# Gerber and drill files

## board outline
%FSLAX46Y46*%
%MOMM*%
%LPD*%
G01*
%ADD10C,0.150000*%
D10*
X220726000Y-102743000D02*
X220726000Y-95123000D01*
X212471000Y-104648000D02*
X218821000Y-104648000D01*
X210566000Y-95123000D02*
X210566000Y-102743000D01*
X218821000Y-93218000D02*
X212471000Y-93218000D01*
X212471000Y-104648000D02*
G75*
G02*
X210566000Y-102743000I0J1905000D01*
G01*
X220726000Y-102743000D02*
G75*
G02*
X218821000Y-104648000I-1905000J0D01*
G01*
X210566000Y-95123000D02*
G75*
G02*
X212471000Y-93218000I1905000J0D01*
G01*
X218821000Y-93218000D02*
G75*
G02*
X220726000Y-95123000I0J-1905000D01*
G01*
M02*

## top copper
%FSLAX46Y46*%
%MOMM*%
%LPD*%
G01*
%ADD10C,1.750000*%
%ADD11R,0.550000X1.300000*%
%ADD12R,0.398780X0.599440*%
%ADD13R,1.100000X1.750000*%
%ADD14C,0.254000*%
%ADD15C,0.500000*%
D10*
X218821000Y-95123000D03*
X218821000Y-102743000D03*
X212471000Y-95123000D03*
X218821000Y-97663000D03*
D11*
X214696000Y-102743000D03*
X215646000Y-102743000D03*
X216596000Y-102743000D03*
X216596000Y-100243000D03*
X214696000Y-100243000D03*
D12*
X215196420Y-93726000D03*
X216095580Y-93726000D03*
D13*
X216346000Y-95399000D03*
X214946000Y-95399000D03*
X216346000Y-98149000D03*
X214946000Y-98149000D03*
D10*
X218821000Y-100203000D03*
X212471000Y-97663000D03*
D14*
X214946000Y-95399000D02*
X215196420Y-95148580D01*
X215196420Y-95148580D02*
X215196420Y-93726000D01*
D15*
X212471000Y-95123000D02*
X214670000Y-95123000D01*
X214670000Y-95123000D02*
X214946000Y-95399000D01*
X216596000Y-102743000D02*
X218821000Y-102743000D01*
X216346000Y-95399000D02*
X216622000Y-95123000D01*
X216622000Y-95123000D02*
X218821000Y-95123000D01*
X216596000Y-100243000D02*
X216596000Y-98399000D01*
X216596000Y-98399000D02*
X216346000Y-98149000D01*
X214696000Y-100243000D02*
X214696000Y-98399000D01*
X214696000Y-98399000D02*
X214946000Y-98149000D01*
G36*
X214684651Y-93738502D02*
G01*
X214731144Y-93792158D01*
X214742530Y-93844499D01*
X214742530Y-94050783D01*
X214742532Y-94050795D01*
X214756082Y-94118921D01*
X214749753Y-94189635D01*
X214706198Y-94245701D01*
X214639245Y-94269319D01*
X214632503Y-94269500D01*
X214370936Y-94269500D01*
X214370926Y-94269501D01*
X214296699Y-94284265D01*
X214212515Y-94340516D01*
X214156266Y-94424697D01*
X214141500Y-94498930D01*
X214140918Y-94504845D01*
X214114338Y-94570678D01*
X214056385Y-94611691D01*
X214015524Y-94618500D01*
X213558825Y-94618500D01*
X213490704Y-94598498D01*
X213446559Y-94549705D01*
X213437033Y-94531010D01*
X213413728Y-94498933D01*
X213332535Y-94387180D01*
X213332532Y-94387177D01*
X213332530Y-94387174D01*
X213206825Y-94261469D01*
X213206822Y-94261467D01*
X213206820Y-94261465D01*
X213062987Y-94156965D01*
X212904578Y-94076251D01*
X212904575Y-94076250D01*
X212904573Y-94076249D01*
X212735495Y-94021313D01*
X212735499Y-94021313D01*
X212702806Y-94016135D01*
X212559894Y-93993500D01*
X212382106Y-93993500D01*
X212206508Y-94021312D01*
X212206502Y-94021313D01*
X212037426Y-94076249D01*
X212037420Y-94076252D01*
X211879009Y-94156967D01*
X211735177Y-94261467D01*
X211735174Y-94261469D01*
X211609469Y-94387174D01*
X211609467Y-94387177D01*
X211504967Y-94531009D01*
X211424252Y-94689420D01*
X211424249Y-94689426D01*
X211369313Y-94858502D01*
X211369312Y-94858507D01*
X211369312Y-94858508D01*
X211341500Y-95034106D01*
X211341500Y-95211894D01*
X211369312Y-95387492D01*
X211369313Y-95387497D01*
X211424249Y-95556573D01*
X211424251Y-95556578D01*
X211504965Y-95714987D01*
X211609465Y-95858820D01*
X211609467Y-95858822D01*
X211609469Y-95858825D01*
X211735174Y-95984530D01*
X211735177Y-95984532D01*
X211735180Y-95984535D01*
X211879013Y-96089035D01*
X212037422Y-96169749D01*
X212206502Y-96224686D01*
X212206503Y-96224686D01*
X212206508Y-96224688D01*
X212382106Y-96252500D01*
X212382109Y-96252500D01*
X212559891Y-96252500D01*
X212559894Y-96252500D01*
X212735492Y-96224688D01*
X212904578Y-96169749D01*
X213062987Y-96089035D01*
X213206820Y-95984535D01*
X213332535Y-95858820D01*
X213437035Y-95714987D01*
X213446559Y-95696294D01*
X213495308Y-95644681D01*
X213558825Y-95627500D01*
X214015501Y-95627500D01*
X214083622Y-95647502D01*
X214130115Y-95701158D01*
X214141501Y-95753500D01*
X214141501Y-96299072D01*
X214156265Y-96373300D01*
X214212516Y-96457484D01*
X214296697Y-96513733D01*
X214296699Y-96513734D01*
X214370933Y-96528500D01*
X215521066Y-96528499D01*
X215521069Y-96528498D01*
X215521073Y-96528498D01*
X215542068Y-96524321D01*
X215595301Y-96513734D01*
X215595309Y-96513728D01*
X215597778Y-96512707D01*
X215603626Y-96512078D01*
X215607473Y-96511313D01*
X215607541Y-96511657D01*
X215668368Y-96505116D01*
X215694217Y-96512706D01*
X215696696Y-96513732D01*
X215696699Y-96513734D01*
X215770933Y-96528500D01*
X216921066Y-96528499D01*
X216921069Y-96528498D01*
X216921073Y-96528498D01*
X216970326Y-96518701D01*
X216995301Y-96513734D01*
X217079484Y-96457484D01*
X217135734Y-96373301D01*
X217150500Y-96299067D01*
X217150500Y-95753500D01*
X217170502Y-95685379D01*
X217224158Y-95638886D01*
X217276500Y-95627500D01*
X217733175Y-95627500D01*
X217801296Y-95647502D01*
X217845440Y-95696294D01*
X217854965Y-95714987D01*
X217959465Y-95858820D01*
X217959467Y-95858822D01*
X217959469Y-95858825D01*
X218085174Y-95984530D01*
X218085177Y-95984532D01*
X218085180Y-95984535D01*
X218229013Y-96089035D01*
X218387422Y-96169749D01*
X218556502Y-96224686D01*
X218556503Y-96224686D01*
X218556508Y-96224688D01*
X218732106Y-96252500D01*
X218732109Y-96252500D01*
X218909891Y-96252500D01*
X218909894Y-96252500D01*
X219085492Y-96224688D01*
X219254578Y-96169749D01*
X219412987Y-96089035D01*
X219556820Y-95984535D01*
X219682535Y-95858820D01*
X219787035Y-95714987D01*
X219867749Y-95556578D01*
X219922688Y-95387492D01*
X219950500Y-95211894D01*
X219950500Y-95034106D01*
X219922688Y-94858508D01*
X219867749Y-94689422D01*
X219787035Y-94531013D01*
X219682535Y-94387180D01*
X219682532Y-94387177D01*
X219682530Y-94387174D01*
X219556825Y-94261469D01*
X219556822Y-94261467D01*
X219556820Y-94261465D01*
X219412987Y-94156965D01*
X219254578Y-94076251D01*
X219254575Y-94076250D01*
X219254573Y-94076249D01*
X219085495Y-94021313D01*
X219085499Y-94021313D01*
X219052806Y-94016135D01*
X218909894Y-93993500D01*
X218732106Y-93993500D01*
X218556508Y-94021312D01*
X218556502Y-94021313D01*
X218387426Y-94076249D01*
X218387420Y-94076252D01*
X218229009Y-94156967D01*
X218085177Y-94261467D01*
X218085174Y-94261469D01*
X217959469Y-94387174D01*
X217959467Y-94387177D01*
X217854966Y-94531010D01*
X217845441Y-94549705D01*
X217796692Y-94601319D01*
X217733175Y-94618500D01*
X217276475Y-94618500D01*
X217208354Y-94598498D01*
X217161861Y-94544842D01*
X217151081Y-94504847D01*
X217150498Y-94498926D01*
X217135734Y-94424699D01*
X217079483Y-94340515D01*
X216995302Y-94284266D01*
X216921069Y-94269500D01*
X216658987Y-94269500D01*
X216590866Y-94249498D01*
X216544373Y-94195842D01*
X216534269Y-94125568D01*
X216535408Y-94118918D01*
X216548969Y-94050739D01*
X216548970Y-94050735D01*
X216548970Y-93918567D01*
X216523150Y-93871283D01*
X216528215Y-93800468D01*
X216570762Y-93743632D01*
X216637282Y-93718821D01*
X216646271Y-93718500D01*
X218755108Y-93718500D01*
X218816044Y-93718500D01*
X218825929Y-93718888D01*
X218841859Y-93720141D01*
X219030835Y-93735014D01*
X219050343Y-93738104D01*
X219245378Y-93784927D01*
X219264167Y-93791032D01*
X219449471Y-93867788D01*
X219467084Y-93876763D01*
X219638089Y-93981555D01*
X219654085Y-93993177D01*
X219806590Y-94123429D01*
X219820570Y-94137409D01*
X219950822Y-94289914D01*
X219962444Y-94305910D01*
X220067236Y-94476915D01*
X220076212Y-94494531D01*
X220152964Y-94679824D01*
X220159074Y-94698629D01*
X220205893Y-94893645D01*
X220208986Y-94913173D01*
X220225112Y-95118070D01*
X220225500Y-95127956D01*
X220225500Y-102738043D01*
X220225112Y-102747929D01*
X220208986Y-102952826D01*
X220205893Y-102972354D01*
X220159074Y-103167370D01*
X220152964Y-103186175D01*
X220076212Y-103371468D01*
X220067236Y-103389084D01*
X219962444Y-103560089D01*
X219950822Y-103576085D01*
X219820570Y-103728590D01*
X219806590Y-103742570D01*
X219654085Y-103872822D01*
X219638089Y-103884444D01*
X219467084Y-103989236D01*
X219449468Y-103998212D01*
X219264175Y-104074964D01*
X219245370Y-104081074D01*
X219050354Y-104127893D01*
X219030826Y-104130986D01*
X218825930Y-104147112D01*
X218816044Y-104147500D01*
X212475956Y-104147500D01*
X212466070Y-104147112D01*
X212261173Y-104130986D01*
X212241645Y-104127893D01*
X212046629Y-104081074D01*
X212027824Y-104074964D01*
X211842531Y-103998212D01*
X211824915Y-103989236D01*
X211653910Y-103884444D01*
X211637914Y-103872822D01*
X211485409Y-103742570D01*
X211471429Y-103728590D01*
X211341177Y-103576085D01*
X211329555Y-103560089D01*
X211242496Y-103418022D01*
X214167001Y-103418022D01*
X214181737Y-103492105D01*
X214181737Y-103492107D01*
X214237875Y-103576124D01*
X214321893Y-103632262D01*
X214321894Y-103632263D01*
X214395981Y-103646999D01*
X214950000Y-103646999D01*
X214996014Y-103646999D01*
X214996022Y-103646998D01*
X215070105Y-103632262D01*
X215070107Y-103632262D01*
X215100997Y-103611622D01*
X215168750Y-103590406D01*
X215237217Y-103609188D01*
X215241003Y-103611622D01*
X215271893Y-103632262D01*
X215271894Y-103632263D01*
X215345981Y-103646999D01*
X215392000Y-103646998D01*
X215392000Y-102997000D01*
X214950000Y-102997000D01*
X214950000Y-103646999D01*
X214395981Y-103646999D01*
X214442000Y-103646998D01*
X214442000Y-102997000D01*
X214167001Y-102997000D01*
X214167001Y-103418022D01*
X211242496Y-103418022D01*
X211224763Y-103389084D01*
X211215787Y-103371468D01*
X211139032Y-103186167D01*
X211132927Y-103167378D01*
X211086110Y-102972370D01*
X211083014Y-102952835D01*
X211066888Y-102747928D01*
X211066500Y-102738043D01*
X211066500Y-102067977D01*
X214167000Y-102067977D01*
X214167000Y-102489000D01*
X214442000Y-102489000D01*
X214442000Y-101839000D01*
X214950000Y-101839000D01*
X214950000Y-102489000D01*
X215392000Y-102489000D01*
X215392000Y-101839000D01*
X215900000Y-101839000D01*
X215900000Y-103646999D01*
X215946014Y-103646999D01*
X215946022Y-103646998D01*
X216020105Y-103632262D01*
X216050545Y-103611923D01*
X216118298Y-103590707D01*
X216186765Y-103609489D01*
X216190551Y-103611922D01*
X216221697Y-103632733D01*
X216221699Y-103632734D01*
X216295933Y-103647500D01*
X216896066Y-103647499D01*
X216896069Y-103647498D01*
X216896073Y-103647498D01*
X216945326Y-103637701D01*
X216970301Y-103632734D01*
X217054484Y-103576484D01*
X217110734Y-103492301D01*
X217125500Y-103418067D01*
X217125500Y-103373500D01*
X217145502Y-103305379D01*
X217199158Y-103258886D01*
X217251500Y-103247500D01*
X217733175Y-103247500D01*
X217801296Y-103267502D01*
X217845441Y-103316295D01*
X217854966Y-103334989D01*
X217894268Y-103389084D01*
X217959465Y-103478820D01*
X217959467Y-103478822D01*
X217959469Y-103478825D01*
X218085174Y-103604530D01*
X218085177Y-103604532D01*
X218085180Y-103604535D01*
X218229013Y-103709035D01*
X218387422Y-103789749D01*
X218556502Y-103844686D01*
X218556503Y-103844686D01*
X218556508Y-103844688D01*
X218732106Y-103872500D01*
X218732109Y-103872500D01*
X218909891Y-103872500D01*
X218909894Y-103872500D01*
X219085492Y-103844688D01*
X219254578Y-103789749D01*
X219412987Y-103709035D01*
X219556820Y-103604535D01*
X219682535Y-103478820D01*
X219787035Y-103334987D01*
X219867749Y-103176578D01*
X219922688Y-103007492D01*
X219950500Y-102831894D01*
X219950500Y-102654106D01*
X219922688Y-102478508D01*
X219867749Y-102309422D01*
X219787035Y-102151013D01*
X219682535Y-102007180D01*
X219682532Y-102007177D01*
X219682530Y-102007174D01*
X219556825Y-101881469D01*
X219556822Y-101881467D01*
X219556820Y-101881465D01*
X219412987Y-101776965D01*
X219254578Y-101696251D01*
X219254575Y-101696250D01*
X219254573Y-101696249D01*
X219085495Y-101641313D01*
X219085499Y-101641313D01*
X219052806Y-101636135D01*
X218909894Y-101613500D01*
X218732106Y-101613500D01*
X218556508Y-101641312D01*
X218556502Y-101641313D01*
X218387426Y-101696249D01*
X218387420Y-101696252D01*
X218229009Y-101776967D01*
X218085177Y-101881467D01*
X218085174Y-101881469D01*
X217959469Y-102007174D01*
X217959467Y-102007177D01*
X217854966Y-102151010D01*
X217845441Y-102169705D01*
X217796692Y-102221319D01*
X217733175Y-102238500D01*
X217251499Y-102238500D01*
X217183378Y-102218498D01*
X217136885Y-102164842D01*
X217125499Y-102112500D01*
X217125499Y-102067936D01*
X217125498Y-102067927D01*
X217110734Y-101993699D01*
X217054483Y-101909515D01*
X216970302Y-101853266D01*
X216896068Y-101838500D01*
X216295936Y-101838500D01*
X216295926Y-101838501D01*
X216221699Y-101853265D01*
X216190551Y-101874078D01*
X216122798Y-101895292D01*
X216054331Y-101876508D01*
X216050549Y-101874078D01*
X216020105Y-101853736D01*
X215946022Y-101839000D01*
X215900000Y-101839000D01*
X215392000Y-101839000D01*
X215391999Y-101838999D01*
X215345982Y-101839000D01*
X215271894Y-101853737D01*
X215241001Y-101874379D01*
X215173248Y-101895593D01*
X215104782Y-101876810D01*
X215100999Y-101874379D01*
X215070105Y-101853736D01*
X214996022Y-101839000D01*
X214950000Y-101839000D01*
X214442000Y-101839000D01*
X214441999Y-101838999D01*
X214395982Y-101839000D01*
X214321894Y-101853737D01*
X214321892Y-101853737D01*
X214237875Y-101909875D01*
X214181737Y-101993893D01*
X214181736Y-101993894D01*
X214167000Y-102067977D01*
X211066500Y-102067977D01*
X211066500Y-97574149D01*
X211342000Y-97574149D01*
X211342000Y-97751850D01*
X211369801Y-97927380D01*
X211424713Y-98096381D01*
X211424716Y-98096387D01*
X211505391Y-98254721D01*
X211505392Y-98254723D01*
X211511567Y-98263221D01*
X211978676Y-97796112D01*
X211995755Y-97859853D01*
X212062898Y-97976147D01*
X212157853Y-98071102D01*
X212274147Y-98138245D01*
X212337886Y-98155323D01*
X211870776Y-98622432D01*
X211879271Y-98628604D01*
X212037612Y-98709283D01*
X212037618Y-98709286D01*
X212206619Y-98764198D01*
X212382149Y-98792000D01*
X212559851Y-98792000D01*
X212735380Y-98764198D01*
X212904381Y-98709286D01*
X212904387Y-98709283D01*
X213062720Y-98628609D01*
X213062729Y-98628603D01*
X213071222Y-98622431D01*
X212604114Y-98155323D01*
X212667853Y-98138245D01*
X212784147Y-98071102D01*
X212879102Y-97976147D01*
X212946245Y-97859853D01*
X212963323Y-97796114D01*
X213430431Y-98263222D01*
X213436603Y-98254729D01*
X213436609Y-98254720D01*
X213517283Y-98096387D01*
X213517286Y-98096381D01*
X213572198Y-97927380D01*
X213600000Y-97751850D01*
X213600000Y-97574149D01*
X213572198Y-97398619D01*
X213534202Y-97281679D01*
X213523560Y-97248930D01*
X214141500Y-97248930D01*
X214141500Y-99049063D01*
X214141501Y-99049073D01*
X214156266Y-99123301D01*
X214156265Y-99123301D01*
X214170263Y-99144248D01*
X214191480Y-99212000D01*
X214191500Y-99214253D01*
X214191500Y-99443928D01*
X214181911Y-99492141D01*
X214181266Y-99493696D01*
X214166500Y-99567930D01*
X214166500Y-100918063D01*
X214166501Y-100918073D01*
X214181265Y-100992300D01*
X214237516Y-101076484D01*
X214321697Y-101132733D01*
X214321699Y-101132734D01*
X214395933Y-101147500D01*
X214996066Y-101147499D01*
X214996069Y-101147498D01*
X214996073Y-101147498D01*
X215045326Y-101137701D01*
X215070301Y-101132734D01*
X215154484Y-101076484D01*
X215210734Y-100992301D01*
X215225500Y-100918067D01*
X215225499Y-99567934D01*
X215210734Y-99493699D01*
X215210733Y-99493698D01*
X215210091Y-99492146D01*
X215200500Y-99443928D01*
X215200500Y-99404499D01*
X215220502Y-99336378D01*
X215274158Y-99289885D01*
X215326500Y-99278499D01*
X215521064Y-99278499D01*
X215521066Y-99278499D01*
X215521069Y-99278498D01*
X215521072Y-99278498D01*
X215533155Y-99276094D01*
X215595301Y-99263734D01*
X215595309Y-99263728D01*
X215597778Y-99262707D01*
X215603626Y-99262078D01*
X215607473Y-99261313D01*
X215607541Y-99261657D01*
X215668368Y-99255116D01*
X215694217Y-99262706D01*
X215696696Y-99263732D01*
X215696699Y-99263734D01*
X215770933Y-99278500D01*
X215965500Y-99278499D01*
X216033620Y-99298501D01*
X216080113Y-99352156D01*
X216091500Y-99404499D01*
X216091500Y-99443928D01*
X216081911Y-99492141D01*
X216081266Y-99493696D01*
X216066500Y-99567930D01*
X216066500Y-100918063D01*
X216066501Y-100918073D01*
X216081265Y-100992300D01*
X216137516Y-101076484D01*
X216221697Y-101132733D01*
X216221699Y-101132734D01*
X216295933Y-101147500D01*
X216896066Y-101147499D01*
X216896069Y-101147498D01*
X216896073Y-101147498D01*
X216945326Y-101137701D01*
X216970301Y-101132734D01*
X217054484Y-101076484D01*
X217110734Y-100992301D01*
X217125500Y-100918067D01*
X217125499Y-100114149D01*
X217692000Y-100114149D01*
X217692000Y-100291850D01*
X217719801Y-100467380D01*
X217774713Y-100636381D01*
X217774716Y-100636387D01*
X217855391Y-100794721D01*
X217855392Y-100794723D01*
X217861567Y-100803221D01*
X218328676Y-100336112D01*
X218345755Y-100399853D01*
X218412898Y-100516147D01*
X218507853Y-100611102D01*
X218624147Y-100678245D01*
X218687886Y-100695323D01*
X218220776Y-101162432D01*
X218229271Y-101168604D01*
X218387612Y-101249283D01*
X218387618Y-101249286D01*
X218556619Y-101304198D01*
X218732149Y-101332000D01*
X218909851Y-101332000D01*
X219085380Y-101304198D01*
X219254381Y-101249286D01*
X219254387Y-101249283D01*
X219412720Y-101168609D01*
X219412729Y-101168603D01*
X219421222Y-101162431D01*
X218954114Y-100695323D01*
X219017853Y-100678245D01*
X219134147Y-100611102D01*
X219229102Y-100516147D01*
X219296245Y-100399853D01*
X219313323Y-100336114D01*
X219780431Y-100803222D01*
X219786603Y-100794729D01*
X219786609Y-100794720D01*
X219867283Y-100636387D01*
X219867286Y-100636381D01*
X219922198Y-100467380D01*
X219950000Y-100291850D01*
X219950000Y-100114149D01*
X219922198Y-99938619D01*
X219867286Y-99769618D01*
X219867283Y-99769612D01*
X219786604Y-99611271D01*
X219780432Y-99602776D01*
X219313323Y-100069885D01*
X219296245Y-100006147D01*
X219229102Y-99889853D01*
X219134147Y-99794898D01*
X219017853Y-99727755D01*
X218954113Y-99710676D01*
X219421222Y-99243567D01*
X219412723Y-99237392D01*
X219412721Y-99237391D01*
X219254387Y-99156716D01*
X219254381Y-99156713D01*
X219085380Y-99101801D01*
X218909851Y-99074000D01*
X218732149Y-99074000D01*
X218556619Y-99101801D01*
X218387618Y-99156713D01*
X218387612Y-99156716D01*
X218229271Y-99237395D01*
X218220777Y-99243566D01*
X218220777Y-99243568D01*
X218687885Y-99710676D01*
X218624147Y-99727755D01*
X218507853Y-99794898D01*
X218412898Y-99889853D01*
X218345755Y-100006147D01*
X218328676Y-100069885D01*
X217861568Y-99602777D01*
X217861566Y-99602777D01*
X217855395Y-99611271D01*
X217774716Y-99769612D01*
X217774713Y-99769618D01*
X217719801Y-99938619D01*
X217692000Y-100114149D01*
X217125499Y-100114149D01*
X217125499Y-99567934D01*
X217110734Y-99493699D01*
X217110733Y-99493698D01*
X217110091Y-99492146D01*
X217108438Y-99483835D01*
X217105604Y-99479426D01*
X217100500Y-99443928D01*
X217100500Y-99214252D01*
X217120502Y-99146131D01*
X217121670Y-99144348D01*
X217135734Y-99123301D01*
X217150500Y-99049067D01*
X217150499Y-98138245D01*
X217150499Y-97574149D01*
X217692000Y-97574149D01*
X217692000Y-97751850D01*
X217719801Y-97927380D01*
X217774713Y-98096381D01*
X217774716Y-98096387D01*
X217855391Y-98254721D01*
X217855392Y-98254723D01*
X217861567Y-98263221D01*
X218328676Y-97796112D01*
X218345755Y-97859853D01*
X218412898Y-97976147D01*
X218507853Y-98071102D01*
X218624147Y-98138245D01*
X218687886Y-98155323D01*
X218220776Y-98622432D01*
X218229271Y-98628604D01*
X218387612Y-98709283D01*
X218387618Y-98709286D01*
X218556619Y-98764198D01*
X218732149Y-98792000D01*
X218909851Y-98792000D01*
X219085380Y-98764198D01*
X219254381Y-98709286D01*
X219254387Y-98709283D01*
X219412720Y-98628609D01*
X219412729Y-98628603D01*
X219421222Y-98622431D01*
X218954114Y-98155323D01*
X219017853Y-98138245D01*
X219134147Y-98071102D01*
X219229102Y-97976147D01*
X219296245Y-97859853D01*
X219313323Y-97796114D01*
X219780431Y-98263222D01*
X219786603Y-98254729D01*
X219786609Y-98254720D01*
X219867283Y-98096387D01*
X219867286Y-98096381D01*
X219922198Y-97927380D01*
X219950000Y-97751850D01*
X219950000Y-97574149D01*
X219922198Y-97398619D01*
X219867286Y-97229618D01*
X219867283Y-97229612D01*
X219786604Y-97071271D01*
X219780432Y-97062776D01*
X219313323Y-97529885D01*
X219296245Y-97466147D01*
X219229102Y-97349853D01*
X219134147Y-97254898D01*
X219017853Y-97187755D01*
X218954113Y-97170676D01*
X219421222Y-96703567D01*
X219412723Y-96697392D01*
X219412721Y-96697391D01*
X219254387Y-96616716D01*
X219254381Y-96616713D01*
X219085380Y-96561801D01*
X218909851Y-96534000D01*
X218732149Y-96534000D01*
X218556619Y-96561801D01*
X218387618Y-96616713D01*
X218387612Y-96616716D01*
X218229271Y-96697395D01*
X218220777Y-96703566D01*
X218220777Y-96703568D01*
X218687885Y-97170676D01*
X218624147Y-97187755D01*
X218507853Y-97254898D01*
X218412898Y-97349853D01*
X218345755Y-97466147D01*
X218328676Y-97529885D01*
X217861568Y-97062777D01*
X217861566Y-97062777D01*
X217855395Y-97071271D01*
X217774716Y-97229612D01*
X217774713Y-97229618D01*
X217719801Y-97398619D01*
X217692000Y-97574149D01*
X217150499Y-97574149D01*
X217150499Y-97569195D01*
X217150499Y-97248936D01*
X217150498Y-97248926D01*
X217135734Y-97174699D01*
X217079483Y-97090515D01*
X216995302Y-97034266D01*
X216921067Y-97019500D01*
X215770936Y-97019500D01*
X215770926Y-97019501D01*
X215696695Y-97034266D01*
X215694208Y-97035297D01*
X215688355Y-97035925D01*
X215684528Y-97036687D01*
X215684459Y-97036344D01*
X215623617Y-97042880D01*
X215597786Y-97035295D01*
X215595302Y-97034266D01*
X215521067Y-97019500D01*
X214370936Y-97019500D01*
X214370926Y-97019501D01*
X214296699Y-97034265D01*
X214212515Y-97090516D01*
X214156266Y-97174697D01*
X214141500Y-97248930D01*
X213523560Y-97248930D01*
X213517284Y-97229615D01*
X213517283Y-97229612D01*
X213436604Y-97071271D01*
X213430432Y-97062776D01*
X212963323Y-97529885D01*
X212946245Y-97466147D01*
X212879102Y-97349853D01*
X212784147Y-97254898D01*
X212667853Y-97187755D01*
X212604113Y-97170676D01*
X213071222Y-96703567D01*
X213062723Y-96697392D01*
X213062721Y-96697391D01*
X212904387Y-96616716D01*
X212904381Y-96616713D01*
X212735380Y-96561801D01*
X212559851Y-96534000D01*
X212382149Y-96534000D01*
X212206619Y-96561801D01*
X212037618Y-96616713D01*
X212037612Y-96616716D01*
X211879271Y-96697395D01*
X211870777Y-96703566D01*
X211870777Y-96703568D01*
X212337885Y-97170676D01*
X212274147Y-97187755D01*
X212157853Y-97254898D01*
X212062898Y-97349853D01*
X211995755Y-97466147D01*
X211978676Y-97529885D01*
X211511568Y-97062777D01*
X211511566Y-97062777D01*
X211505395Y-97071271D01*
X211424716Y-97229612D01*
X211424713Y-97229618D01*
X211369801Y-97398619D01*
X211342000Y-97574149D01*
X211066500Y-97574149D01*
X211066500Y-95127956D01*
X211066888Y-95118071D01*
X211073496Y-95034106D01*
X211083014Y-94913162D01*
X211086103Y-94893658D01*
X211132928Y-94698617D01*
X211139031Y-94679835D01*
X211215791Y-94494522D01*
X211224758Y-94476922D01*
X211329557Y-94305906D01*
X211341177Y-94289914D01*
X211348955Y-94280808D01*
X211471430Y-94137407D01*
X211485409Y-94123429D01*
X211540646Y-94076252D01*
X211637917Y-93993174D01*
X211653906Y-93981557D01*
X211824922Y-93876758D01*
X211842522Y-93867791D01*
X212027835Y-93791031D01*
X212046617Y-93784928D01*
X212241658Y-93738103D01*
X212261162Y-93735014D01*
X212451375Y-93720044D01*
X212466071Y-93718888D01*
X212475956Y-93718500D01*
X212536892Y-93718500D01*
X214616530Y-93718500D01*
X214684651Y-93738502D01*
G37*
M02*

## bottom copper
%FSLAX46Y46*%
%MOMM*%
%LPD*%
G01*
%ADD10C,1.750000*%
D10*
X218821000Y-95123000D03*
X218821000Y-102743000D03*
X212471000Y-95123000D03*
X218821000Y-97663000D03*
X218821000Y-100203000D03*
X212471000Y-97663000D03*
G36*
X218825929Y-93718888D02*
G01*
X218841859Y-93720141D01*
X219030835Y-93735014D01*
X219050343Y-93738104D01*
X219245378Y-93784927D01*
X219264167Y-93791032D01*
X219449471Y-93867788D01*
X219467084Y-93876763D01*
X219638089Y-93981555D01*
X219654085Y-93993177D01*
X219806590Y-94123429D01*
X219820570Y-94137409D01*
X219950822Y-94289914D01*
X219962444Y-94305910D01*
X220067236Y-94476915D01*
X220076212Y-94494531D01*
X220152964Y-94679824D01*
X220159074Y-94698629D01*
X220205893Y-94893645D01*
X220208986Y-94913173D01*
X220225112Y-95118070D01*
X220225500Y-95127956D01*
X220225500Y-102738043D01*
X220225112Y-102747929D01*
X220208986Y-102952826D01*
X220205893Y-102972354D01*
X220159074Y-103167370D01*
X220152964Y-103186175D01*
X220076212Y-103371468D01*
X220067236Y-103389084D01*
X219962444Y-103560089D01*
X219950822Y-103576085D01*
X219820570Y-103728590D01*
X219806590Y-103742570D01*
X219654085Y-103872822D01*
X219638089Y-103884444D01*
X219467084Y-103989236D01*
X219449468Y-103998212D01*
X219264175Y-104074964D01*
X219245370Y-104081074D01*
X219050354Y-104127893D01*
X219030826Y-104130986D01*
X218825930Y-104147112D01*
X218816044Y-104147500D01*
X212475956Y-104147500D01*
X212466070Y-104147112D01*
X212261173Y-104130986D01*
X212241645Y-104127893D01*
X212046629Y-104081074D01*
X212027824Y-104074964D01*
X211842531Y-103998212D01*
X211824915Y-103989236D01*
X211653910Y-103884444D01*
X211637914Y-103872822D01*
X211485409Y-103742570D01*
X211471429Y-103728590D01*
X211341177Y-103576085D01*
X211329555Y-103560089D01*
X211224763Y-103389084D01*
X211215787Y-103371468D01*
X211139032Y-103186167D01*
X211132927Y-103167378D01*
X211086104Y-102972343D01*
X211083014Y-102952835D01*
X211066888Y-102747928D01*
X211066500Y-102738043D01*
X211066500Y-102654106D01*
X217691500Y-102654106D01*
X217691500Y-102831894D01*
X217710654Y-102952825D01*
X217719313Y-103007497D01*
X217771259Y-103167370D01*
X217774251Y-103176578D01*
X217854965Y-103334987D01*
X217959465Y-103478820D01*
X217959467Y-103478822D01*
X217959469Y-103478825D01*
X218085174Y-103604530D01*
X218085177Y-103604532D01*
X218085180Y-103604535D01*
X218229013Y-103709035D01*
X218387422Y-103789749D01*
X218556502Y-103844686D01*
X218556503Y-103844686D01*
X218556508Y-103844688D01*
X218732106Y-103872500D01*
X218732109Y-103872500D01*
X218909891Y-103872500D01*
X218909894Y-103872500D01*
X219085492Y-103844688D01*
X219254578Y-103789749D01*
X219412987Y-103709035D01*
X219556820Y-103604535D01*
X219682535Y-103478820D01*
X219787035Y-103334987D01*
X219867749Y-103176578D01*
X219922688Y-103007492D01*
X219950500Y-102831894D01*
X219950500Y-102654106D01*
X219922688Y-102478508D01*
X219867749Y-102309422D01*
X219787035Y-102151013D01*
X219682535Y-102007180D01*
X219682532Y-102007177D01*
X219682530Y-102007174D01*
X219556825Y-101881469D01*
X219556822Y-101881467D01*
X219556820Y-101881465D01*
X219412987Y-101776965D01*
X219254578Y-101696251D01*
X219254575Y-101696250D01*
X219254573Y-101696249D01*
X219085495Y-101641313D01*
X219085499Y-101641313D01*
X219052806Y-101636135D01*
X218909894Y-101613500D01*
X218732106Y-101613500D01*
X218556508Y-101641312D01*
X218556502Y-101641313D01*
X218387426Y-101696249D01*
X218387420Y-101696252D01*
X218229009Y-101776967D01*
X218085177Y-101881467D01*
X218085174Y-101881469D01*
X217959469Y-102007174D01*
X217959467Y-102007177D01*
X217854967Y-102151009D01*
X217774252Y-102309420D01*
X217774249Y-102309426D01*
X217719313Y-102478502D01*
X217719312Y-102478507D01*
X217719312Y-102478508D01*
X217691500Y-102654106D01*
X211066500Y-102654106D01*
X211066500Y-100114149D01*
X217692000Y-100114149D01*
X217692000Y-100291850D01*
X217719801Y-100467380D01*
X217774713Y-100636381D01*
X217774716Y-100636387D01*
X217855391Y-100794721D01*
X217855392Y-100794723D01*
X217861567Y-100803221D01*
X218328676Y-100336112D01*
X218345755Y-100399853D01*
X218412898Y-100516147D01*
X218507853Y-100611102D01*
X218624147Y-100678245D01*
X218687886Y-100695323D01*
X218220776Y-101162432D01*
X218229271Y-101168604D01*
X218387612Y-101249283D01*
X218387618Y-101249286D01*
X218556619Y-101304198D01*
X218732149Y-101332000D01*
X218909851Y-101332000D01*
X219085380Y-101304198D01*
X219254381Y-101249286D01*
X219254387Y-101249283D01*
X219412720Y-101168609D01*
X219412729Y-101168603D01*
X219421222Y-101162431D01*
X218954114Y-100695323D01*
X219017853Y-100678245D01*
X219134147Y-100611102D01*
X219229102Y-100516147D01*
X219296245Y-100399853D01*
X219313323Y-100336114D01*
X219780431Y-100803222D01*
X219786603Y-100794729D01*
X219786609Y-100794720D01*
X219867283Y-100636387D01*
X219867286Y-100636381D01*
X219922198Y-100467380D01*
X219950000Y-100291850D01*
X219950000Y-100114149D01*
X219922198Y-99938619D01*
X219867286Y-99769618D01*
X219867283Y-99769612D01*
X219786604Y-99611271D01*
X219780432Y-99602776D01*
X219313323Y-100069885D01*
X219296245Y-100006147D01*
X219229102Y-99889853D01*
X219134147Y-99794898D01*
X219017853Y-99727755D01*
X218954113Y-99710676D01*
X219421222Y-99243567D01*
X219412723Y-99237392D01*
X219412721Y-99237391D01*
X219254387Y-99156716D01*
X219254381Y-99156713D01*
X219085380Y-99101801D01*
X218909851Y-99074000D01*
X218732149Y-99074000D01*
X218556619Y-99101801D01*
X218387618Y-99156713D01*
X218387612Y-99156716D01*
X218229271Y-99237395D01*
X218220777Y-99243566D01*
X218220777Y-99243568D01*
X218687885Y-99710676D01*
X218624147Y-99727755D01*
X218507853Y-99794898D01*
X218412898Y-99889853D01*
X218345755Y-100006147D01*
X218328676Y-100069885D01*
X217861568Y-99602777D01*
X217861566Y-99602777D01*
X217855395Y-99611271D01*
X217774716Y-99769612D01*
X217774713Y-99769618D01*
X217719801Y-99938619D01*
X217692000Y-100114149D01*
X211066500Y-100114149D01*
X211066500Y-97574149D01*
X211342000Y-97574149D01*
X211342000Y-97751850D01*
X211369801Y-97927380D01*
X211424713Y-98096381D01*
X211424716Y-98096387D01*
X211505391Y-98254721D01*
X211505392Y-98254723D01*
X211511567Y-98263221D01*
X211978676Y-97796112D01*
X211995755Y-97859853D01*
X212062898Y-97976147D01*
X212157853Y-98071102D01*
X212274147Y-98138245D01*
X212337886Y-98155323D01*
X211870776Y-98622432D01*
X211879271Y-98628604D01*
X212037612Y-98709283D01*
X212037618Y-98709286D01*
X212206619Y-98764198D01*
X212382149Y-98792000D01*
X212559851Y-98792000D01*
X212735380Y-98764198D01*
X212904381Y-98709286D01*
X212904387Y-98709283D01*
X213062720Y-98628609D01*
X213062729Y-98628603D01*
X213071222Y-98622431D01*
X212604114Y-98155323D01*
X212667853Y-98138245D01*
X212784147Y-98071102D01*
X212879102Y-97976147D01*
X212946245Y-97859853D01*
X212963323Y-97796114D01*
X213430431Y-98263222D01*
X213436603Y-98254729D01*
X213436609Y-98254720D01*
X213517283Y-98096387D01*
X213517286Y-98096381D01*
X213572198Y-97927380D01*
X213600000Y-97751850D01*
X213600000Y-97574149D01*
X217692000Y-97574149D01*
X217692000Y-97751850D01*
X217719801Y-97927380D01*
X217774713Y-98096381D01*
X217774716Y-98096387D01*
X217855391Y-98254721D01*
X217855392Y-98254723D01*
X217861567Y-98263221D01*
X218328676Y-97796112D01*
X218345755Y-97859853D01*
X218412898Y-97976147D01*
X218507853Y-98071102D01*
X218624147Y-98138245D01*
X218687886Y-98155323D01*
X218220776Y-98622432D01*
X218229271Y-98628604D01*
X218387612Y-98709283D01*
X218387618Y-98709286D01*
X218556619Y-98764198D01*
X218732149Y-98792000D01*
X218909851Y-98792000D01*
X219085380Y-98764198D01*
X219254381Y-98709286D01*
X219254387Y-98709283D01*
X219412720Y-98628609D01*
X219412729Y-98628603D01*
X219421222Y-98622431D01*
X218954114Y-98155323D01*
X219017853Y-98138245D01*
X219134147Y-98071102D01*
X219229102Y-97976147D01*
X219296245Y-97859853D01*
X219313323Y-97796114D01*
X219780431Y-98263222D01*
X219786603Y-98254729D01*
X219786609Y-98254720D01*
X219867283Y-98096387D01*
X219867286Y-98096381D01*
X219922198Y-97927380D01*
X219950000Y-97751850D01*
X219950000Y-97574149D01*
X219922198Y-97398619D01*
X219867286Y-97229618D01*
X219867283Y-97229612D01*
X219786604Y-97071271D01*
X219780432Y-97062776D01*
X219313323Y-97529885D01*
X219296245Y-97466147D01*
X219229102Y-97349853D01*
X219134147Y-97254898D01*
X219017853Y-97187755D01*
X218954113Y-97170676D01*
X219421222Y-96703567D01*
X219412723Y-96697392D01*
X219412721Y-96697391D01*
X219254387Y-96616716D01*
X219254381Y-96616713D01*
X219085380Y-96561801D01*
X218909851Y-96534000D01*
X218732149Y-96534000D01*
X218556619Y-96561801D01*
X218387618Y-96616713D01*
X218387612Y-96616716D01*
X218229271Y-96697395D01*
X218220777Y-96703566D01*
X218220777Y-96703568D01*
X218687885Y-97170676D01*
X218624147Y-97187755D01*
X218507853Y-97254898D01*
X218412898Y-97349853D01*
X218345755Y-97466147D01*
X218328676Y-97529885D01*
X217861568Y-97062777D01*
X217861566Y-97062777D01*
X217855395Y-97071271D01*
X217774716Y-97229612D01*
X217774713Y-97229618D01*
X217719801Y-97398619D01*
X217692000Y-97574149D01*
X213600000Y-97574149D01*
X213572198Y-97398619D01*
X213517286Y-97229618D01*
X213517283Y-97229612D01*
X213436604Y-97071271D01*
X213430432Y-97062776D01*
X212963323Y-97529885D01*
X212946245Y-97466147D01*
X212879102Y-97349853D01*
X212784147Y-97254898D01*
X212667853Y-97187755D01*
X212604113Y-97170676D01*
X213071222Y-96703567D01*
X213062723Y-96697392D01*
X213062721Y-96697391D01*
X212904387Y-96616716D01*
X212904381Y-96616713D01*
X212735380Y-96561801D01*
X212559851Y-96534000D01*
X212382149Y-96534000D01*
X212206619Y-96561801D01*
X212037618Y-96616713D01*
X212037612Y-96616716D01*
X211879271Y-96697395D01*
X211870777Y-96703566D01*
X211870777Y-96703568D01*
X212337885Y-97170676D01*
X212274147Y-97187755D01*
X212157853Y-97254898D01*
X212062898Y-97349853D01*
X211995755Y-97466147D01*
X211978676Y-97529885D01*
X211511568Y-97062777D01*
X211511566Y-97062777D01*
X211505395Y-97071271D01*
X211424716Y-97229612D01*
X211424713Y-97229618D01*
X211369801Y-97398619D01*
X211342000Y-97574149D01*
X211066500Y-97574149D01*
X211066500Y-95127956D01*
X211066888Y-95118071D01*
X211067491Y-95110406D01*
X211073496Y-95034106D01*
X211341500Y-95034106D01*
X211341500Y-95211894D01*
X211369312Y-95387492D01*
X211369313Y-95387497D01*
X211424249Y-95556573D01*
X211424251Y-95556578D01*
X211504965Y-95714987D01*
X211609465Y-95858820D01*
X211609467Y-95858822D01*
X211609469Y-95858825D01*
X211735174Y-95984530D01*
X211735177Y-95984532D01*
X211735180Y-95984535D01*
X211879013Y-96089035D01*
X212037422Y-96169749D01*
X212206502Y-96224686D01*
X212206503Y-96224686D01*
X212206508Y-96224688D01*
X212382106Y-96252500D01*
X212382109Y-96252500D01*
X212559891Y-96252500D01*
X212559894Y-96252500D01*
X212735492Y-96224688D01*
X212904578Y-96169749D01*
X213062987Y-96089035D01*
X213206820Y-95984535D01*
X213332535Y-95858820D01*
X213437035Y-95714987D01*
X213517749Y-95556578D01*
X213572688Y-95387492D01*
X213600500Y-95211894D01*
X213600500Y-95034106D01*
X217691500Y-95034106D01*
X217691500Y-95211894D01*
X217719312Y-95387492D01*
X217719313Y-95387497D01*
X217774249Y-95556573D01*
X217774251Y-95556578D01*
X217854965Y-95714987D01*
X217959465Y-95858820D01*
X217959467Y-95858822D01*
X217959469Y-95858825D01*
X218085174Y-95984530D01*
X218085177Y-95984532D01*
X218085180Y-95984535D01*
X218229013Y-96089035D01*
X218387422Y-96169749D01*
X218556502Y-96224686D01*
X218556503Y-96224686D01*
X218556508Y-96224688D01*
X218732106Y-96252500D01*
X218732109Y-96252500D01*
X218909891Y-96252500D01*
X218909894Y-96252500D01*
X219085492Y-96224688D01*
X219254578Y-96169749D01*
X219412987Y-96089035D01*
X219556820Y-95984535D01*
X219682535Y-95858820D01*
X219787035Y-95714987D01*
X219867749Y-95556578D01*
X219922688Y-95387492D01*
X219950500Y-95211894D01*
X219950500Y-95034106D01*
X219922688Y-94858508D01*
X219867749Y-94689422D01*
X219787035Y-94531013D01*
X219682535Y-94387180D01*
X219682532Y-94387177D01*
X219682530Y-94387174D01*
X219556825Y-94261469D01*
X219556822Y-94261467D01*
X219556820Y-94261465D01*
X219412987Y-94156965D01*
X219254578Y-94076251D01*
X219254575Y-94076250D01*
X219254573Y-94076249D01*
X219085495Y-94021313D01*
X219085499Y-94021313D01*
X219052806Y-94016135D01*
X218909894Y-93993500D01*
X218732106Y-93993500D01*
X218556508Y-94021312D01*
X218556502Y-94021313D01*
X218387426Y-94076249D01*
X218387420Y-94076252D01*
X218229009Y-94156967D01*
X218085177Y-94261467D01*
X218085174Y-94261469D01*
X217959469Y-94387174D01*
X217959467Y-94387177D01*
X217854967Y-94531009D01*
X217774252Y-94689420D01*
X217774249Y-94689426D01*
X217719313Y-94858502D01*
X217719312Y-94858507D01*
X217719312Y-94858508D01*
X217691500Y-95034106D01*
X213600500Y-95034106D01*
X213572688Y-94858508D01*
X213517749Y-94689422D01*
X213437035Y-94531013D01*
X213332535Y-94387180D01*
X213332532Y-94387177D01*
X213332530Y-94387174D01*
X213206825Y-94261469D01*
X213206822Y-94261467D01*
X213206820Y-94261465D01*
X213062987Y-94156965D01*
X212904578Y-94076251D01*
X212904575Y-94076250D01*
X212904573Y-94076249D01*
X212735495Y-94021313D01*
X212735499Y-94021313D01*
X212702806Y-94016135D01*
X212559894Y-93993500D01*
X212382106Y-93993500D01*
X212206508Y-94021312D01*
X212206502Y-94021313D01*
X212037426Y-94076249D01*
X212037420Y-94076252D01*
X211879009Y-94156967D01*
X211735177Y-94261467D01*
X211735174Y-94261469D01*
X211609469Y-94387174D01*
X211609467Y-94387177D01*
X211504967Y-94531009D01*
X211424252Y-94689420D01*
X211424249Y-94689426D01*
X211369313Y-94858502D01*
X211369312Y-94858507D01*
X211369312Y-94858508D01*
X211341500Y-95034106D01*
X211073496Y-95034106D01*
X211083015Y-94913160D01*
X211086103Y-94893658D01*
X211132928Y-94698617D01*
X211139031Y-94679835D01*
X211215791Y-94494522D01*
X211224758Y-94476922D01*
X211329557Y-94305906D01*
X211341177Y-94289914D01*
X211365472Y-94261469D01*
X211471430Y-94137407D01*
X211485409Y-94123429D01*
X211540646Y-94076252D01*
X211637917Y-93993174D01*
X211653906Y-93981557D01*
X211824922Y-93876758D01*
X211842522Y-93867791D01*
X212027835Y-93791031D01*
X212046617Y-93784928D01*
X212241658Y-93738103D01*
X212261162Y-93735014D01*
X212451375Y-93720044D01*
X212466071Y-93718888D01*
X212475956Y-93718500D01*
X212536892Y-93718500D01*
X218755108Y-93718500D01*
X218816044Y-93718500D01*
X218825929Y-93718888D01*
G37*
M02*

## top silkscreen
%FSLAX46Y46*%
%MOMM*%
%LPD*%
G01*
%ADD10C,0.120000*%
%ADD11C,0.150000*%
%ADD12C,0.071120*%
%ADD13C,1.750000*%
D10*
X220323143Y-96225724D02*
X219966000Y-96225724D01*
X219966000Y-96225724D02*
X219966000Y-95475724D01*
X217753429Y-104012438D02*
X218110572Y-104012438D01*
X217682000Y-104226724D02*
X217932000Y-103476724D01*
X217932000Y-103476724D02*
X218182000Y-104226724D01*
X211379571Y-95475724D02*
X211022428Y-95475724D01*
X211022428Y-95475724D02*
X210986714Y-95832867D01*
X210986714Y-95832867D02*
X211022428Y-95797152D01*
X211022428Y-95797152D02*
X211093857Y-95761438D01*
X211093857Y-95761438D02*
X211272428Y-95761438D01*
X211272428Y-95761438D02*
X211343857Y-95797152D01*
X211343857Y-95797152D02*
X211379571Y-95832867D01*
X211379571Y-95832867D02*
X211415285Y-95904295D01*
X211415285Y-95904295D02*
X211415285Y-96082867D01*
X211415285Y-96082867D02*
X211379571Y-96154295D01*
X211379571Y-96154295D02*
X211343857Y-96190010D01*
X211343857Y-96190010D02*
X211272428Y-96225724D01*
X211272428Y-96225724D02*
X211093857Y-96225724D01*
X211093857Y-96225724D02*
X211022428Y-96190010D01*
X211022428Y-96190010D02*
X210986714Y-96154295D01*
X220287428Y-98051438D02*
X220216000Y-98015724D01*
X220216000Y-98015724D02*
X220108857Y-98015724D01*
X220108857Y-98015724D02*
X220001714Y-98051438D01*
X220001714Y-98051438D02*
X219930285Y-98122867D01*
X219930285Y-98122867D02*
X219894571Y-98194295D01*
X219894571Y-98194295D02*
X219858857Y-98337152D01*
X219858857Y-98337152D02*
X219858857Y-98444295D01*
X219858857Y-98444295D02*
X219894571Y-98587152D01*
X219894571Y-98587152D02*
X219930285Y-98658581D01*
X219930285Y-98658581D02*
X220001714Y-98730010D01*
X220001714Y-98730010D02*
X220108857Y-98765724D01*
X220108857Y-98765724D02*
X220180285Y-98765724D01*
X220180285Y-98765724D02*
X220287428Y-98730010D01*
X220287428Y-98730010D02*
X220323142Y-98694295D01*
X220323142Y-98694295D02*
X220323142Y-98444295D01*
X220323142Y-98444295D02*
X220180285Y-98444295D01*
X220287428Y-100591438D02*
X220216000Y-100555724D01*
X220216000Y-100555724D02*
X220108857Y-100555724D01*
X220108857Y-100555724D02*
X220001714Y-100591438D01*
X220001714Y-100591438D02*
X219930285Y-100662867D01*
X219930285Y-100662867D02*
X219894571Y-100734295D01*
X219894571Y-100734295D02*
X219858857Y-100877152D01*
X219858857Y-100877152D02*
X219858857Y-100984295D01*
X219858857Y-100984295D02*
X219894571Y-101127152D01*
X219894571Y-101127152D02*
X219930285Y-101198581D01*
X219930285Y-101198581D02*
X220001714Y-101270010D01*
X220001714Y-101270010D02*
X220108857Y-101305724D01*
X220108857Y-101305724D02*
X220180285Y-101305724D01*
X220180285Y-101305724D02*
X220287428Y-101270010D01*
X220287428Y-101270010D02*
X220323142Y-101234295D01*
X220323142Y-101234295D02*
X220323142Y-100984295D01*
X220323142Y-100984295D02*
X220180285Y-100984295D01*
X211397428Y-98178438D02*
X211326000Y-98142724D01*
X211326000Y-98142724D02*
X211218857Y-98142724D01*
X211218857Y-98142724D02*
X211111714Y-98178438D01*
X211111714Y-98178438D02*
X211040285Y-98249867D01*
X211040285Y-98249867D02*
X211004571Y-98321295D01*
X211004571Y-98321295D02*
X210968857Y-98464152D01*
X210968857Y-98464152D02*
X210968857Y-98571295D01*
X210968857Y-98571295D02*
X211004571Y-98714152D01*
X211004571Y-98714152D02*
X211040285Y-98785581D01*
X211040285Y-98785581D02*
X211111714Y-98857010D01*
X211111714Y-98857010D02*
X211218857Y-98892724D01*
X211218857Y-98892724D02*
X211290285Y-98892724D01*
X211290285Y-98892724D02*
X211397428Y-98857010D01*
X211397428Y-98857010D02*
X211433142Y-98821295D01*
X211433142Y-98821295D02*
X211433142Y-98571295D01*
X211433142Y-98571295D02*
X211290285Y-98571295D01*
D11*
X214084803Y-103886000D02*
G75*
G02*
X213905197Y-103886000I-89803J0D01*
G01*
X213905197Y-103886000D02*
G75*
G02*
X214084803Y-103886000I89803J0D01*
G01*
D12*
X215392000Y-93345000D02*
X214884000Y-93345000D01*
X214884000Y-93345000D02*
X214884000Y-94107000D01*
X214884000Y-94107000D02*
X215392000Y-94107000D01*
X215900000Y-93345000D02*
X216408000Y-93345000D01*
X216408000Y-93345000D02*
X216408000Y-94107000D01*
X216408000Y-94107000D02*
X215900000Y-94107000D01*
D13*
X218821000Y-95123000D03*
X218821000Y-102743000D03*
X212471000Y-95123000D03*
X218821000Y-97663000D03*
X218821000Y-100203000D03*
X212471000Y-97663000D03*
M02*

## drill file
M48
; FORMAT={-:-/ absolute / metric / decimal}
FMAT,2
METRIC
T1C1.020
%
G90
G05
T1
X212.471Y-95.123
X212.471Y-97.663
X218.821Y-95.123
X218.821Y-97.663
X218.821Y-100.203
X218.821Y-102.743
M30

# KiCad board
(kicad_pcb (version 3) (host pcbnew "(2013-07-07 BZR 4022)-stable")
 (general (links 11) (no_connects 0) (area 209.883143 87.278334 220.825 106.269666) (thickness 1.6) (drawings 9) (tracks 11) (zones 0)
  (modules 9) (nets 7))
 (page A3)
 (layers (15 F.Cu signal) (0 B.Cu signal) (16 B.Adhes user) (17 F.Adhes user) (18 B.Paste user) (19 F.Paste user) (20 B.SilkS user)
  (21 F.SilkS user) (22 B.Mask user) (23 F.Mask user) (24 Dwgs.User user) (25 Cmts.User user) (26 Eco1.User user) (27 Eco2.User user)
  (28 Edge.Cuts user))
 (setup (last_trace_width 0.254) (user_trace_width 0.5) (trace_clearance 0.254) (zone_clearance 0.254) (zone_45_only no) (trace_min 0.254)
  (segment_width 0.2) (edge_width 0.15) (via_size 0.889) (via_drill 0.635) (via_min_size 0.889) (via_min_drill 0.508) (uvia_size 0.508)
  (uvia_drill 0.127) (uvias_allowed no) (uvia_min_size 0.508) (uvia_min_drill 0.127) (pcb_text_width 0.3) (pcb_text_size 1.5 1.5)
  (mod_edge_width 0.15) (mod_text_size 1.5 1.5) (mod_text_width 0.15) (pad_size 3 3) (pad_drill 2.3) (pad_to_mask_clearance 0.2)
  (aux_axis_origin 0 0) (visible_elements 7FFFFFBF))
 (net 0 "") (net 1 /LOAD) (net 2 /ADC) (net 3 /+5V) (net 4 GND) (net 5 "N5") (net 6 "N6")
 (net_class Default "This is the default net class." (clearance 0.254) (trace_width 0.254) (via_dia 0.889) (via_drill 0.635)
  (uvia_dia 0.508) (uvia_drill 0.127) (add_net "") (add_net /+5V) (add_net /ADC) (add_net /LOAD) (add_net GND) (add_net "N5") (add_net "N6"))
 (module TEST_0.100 (layer F.Cu) (at 218.821 95.123)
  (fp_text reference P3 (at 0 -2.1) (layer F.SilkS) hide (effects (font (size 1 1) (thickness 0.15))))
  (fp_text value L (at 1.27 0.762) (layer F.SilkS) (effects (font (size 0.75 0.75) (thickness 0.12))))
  (pad 1 thru_hole circle (at 0 0) (size 1.75 1.75) (drill 1.02) (layers *.Cu *.Mask F.SilkS) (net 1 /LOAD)))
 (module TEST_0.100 (layer F.Cu) (at 218.821 102.743)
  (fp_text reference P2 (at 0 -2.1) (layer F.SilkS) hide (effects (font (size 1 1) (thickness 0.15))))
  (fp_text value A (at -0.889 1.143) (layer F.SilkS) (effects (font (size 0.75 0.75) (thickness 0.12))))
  (pad 1 thru_hole circle (at 0 0) (size 1.75 1.75) (drill 1.02) (layers *.Cu *.Mask F.SilkS) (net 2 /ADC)))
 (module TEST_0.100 (layer F.Cu) (at 212.471 95.123)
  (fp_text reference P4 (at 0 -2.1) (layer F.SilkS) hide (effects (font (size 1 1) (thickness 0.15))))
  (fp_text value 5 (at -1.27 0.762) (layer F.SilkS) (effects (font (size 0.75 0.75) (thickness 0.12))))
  (pad 1 thru_hole circle (at 0 0) (size 1.75 1.75) (drill 1.02) (layers *.Cu *.Mask F.SilkS) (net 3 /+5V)))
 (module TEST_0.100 (layer F.Cu) (at 218.821 97.663)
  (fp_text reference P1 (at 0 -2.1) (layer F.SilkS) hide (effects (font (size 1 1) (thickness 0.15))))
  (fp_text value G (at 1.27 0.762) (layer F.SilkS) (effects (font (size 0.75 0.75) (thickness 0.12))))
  (pad 1 thru_hole circle (at 0 0) (size 1.75 1.75) (drill 1.02) (layers *.Cu *.Mask F.SilkS) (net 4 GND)))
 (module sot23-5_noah (layer F.Cu) (at 215.646 102.743 90)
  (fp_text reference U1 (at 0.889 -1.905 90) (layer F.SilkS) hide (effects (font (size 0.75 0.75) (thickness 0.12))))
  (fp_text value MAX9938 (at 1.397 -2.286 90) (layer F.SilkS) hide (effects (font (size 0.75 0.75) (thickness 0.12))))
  (fp_circle (center -1.143 -1.651) (end -1.0795 -1.5875) (layer F.SilkS) (width 0.15))
  (pad 1 smd rect (at 0 -0.95 90) (size 1.3 0.55) (layers F.Cu F.Paste F.Mask) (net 4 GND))
  (pad 2 smd rect (at 0 0 90) (size 1.3 0.55) (layers F.Cu F.Paste F.Mask) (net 4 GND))
  (pad 3 smd rect (at 0 0.95 90) (size 1.3 0.55) (layers F.Cu F.Paste F.Mask) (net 2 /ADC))
  (pad 4 smd rect (at 2.5 0.95 90) (size 1.3 0.55) (layers F.Cu F.Paste F.Mask) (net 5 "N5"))
  (pad 5 smd rect (at 2.5 -0.95 90) (size 1.3 0.55) (layers F.Cu F.Paste F.Mask) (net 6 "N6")))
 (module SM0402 (layer F.Cu) (at 215.646 93.726)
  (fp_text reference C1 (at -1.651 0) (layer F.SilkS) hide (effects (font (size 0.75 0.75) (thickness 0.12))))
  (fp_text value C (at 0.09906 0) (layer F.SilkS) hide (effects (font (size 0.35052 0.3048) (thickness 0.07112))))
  (fp_line (start -0.254 -0.381) (end -0.762 -0.381) (layer F.SilkS) (width 0.07112))
  (fp_line (start -0.762 -0.381) (end -0.762 0.381) (layer F.SilkS) (width 0.07112))
  (fp_line (start -0.762 0.381) (end -0.254 0.381) (layer F.SilkS) (width 0.07112))
  (fp_line (start 0.254 -0.381) (end 0.762 -0.381) (layer F.SilkS) (width 0.07112))
  (fp_line (start 0.762 -0.381) (end 0.762 0.381) (layer F.SilkS) (width 0.07112))
  (fp_line (start 0.762 0.381) (end 0.254 0.381) (layer F.SilkS) (width 0.07112))
  (pad 1 smd rect (at -0.44958 0) (size 0.39878 0.59944) (layers F.Cu F.Paste F.Mask) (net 3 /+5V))
  (pad 2 smd rect (at 0.44958 0) (size 0.39878 0.59944) (layers F.Cu F.Paste F.Mask) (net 4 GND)))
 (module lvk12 (layer F.Cu) (at 215.646 96.774 270)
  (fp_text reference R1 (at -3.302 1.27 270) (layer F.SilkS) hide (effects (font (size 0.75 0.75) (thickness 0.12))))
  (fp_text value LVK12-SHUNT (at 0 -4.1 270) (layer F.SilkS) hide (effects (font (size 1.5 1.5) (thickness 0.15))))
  (pad 1 smd rect (at -1.375 -0.7 270) (size 1.75 1.1) (layers F.Cu F.Paste F.Mask) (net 1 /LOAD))
  (pad 2 smd rect (at -1.375 0.7 270) (size 1.75 1.1) (layers F.Cu F.Paste F.Mask) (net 3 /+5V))
  (pad 4 smd rect (at 1.375 -0.7 270) (size 1.75 1.1) (layers F.Cu F.Paste F.Mask) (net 5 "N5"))
  (pad 3 smd rect (at 1.375 0.7 270) (size 1.75 1.1) (layers F.Cu F.Paste F.Mask) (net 6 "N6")))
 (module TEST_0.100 (layer F.Cu) (at 218.821 100.203)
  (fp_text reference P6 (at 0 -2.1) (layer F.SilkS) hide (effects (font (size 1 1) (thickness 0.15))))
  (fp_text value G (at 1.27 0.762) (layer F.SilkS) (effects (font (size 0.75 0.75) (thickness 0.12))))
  (pad 1 thru_hole circle (at 0 0) (size 1.75 1.75) (drill 1.02) (layers *.Cu *.Mask F.SilkS) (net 4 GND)))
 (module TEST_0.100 (layer F.Cu) (at 212.471 97.663)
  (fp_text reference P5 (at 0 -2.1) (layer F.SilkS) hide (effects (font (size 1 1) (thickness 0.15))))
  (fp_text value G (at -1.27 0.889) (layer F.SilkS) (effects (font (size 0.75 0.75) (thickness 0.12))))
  (pad 1 thru_hole circle (at 0 0) (size 1.75 1.75) (drill 1.02) (layers *.Cu *.Mask F.SilkS) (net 4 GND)))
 (gr_line (start 220.726 102.743) (end 220.726 95.123) (angle 90) (layer Edge.Cuts) (width 0.15))
 (gr_line (start 212.471 104.648) (end 218.821 104.648) (angle 90) (layer Edge.Cuts) (width 0.15))
 (gr_line (start 210.566 95.123) (end 210.566 102.743) (angle 90) (layer Edge.Cuts) (width 0.15))
 (gr_line (start 218.821 93.218) (end 212.471 93.218) (angle 90) (layer Edge.Cuts) (width 0.15))
 (gr_arc (start 212.471 102.743) (end 212.471 104.648) (angle 90) (layer Edge.Cuts) (width 0.15))
 (gr_arc (start 218.821 102.743) (end 220.726 102.743) (angle 90) (layer Edge.Cuts) (width 0.15))
 (gr_arc (start 212.471 95.123) (end 210.566 95.123) (angle 90) (layer Edge.Cuts) (width 0.15))
 (gr_arc (start 218.821 95.123) (end 218.821 93.218) (angle 90) (layer Edge.Cuts) (width 0.15))
 (segment (start 214.946 95.399) (end 215.19642 95.14858) (width 0.254) (layer F.Cu) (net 3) (status C00000))
 (segment (start 215.19642 95.14858) (end 215.19642 93.726) (width 0.254) (layer F.Cu) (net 3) (status C00000))
 (segment (start 212.471 95.123) (end 214.67 95.123) (width 0.5) (layer F.Cu) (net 3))
 (segment (start 214.67 95.123) (end 214.946 95.399) (width 0.5) (layer F.Cu) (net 3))
 (segment (start 216.596 102.743) (end 218.821 102.743) (width 0.5) (layer F.Cu) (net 2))
 (segment (start 216.346 95.399) (end 216.622 95.123) (width 0.5) (layer F.Cu) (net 1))
 (segment (start 216.622 95.123) (end 218.821 95.123) (width 0.5) (layer F.Cu) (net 1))
 (segment (start 216.596 100.243) (end 216.596 98.399) (width 0.5) (layer F.Cu) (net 5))
 (segment (start 216.596 98.399) (end 216.346 98.149) (width 0.5) (layer F.Cu) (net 5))
 (segment (start 214.696 100.243) (end 214.696 98.399) (width 0.5) (layer F.Cu) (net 6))
 (segment (start 214.696 98.399) (end 214.946 98.149) (width 0.5) (layer F.Cu) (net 6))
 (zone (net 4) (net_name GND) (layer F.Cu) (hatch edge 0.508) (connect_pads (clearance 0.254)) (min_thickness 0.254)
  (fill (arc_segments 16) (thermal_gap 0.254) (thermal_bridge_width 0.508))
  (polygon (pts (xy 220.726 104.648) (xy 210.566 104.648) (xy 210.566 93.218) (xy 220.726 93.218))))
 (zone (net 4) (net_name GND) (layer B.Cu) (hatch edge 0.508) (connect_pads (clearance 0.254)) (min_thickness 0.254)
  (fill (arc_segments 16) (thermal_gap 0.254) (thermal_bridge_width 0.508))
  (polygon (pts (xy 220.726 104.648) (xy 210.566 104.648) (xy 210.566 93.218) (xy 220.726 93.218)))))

